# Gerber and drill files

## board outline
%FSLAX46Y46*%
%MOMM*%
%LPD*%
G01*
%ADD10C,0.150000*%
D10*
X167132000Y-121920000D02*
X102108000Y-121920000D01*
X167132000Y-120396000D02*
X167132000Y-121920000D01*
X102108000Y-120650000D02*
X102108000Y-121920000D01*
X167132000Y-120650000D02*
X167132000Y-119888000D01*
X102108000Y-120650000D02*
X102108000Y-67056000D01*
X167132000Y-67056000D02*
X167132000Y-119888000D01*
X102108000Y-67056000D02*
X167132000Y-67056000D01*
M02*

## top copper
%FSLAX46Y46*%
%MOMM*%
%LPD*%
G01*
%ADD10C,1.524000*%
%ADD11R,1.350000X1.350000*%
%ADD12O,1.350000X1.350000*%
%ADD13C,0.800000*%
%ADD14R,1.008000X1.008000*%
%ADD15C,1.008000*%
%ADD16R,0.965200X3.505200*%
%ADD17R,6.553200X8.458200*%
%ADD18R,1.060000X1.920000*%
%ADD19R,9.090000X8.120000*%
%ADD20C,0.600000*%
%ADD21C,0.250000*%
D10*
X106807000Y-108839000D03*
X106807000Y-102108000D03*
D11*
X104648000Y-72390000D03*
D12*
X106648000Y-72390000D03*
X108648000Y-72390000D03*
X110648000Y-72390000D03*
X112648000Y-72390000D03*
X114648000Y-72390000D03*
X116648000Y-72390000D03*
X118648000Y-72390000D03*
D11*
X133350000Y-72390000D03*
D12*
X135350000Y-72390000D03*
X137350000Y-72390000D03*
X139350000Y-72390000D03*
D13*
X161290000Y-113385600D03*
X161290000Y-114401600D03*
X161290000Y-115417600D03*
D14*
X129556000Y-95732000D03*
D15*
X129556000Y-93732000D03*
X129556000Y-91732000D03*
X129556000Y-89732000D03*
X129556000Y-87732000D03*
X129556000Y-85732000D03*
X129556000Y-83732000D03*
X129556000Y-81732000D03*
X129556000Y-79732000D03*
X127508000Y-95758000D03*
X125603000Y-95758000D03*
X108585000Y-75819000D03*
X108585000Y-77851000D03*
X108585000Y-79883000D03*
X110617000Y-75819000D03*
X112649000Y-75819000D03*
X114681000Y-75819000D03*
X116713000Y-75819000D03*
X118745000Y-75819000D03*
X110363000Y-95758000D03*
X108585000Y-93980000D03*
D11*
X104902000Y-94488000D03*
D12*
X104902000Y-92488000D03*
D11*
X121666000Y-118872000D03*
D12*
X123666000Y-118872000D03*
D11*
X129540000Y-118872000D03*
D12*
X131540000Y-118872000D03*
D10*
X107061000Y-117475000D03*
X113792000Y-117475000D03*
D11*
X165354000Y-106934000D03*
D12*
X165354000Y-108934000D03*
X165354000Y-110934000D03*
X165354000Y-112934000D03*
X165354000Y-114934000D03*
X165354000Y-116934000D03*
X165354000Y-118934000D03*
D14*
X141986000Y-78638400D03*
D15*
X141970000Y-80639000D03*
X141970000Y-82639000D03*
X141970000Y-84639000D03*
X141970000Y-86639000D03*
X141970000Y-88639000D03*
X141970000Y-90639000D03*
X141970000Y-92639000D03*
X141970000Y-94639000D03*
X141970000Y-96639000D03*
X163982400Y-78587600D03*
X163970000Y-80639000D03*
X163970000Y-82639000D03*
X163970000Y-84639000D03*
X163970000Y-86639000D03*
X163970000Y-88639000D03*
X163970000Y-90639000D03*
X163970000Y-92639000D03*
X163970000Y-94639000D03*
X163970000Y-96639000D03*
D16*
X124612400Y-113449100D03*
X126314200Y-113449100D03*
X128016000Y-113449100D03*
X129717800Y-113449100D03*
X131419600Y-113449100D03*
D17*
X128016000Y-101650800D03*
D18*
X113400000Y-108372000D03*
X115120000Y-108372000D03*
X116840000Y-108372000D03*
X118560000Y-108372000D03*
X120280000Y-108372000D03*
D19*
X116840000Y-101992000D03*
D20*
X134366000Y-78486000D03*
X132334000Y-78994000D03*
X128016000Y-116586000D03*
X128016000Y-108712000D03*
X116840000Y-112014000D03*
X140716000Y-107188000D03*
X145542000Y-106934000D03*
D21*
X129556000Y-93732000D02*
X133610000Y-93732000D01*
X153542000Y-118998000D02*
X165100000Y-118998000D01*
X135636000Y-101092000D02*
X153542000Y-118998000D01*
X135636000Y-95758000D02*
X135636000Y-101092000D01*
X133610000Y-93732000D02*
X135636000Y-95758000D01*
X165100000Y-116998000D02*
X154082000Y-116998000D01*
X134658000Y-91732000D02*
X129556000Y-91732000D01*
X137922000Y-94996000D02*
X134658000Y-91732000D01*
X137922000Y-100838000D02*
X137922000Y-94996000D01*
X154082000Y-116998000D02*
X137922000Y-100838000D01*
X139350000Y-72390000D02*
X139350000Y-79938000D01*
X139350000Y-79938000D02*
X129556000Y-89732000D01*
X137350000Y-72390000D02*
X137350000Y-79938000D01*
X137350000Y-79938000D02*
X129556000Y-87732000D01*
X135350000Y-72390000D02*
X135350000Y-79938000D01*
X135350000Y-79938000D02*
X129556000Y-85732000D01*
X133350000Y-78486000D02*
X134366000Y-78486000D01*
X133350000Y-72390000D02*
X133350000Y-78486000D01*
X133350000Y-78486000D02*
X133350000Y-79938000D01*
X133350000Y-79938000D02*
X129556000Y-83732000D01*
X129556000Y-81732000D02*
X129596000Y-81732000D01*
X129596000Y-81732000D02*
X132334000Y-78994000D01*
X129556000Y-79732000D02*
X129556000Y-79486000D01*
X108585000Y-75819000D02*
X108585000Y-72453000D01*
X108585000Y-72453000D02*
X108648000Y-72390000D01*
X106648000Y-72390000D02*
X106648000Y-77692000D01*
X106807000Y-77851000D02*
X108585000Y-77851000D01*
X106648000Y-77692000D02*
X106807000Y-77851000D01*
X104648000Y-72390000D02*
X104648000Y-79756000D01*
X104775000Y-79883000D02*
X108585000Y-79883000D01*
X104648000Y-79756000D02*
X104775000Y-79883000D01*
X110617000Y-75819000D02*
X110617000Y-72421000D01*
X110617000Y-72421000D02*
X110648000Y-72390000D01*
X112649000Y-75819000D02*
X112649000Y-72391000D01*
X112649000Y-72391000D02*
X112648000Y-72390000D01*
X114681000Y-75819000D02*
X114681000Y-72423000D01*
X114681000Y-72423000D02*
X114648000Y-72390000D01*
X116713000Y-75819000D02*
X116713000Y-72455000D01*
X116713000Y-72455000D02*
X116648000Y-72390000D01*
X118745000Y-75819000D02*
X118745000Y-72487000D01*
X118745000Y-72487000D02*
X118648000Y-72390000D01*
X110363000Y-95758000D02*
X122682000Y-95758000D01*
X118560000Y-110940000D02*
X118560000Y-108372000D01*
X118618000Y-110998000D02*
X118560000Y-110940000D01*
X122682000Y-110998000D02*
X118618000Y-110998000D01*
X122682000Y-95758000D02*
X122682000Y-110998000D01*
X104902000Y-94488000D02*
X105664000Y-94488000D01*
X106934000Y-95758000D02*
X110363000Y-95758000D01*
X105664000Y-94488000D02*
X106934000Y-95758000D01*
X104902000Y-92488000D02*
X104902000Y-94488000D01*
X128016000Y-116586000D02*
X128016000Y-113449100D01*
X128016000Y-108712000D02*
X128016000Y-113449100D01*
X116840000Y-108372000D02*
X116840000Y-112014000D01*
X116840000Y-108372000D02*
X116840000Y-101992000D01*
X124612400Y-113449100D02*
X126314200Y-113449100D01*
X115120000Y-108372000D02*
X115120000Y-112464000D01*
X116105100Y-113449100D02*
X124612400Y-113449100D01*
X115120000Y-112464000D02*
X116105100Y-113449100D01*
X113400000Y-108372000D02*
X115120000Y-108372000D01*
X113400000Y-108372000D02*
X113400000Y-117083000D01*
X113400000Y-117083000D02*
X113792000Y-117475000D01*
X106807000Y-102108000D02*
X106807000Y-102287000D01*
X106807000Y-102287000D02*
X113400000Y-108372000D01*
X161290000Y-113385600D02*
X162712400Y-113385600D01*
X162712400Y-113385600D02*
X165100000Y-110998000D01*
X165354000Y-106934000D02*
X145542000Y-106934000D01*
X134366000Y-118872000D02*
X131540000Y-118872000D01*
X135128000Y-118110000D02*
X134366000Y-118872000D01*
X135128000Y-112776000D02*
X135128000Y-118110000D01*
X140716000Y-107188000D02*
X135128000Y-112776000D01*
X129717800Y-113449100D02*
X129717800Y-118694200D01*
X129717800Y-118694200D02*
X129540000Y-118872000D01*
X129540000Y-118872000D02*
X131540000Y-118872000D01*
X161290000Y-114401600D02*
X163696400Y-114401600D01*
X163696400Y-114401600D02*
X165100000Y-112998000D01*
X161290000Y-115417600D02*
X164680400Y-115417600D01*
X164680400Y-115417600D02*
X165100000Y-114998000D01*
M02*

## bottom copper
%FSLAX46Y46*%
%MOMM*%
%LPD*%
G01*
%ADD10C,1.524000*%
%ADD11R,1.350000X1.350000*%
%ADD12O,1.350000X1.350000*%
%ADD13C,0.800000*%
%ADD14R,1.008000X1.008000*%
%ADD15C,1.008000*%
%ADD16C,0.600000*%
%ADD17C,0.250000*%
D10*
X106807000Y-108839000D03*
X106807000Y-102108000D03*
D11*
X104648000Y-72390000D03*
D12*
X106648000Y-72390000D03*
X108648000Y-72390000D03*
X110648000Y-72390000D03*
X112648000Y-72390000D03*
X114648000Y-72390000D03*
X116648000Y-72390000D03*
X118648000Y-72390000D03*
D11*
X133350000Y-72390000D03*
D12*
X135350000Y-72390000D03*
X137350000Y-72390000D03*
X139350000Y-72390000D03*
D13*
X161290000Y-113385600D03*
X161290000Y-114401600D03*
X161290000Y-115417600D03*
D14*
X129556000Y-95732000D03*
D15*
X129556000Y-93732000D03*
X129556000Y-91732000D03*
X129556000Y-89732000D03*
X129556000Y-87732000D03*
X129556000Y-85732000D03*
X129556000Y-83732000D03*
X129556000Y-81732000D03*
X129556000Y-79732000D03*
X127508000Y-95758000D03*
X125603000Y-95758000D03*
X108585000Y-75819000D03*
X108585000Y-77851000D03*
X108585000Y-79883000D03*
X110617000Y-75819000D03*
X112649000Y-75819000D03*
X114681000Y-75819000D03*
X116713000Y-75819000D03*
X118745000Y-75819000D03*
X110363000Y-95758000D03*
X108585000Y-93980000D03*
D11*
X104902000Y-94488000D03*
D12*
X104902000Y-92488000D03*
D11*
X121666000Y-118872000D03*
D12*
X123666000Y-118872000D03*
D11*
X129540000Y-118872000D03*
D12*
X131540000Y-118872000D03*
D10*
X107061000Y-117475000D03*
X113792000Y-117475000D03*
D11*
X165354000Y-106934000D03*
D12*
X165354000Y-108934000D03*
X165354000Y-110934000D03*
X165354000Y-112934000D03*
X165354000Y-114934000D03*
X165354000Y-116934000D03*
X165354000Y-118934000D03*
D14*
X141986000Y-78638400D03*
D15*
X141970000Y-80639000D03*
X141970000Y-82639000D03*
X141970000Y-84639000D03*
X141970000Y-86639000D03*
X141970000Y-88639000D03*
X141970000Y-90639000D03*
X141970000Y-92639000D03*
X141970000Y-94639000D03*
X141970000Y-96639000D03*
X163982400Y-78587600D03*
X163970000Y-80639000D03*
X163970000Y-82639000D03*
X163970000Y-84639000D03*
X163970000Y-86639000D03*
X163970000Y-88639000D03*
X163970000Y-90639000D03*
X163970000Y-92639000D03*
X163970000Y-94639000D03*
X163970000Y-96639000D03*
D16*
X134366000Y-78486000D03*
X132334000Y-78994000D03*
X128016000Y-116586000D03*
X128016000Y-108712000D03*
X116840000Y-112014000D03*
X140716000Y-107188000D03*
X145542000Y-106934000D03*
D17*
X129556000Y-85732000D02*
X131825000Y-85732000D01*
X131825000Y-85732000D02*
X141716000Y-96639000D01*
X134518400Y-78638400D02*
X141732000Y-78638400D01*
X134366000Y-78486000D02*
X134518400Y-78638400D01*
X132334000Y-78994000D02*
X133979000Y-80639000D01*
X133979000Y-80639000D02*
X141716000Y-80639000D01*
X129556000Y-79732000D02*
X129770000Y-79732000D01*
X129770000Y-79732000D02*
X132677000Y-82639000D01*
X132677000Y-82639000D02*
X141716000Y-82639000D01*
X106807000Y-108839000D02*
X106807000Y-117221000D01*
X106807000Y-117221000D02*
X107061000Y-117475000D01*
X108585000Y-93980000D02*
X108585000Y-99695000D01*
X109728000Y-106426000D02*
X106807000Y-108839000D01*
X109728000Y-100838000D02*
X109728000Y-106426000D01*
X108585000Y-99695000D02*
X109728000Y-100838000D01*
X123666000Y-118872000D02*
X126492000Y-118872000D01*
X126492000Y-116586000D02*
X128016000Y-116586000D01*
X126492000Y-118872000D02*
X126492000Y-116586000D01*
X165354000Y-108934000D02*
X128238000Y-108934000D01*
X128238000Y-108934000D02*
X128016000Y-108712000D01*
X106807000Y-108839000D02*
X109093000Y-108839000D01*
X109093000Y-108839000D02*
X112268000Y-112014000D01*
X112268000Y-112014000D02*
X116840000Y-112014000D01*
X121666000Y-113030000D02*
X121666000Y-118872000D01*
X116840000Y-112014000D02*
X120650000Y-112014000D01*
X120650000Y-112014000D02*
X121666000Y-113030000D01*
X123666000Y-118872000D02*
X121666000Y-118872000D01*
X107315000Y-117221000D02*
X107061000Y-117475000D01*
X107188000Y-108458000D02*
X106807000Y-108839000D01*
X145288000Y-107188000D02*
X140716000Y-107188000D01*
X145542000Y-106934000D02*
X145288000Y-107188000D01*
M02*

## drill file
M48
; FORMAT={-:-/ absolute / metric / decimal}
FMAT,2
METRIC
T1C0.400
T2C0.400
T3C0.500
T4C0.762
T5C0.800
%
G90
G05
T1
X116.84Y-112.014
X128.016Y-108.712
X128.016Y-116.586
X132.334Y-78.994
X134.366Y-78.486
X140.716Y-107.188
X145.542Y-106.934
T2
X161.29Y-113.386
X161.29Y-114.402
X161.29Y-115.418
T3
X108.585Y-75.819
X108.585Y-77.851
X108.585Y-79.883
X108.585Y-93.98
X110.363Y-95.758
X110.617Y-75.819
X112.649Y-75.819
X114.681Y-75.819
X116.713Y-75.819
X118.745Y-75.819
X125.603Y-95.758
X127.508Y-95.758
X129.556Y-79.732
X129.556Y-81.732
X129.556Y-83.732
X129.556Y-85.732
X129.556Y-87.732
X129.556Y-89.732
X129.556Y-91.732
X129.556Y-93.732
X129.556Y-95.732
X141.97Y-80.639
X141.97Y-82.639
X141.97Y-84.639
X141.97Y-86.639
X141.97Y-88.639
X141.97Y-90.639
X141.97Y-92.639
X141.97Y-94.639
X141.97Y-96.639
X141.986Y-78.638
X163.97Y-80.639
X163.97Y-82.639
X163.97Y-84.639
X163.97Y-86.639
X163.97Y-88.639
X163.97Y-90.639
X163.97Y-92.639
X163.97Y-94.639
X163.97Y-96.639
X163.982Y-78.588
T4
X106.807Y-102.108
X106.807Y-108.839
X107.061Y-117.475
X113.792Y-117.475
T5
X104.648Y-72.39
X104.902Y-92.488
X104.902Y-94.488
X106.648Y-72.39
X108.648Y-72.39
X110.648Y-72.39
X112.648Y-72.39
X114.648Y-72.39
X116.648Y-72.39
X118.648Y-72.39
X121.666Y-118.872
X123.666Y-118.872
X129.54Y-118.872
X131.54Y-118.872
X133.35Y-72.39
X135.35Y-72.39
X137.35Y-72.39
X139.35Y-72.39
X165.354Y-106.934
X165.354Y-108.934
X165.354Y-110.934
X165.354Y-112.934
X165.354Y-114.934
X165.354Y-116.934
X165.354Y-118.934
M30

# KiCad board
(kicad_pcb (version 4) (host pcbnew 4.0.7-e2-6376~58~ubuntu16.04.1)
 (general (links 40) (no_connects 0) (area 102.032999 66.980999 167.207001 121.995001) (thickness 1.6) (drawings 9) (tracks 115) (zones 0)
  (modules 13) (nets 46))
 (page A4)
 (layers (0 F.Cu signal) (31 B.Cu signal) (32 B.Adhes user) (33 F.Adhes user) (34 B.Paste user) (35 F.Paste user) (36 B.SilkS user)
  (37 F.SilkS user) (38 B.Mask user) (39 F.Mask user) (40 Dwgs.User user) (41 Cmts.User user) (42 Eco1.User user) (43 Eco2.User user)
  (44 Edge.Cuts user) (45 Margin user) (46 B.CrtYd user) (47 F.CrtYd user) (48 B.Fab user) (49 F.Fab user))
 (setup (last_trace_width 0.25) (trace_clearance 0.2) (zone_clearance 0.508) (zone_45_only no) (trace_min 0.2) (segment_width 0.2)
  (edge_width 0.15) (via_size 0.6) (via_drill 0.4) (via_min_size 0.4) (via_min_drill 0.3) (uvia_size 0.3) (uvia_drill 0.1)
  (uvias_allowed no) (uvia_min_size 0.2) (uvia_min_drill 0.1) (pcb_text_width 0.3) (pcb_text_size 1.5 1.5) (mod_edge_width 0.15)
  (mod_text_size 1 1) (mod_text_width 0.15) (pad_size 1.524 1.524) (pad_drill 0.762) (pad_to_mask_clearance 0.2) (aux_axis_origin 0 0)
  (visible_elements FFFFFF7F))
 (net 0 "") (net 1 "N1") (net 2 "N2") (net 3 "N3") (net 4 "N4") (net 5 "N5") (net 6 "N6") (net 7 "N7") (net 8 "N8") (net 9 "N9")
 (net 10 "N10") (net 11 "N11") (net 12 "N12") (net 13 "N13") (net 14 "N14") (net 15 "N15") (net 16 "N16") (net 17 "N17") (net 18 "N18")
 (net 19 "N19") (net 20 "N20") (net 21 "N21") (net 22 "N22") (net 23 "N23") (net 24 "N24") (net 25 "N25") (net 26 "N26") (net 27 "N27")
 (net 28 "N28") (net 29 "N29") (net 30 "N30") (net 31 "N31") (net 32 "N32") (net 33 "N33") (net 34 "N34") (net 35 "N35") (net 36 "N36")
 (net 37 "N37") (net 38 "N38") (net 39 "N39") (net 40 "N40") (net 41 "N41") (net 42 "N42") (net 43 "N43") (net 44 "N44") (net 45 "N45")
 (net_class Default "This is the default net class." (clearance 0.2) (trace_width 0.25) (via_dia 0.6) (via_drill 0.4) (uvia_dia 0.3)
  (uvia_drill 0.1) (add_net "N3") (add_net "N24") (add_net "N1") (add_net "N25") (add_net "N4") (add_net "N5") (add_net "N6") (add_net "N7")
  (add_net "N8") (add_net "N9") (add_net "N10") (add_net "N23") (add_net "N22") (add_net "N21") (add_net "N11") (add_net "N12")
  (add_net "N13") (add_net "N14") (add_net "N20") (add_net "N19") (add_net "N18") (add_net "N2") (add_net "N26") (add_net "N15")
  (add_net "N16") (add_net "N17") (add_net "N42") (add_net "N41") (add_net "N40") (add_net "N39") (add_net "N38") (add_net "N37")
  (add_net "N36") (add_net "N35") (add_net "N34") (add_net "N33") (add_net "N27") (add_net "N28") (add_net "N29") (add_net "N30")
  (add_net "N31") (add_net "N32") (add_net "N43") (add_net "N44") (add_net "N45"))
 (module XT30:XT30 (layer F.Cu) (at 100.838 107.442 90)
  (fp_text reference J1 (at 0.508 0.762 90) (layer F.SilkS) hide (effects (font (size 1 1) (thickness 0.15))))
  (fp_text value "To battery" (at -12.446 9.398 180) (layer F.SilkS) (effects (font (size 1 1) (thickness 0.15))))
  (pad 1 thru_hole circle (at -1.397 5.969 90) (size 1.524 1.524) (drill 0.762) (layers *.Cu *.Mask) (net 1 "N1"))
  (pad 2 thru_hole circle (at 5.334 5.969 90) (size 1.524 1.524) (drill 0.762) (layers *.Cu *.Mask) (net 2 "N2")))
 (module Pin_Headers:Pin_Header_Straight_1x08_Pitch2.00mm (layer F.Cu) (at 104.648 72.39 90)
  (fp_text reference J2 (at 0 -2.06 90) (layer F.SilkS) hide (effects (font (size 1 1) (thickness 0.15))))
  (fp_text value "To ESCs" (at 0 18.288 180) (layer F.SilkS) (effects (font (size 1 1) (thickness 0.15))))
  (pad 1 thru_hole rect (at 0 0 90) (size 1.35 1.35) (drill 0.8) (layers *.Cu *.Mask) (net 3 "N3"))
  (pad 2 thru_hole oval (at 0 2 90) (size 1.35 1.35) (drill 0.8) (layers *.Cu *.Mask) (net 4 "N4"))
  (pad 3 thru_hole oval (at 0 4 90) (size 1.35 1.35) (drill 0.8) (layers *.Cu *.Mask) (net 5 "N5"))
  (pad 4 thru_hole oval (at 0 6 90) (size 1.35 1.35) (drill 0.8) (layers *.Cu *.Mask) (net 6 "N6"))
  (pad 5 thru_hole oval (at 0 8 90) (size 1.35 1.35) (drill 0.8) (layers *.Cu *.Mask) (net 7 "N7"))
  (pad 6 thru_hole oval (at 0 10 90) (size 1.35 1.35) (drill 0.8) (layers *.Cu *.Mask) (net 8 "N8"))
  (pad 7 thru_hole oval (at 0 12 90) (size 1.35 1.35) (drill 0.8) (layers *.Cu *.Mask) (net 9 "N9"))
  (pad 8 thru_hole oval (at 0 14 90) (size 1.35 1.35) (drill 0.8) (layers *.Cu *.Mask) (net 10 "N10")))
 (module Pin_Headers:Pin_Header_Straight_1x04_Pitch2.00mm (layer F.Cu) (at 133.35 72.39 90)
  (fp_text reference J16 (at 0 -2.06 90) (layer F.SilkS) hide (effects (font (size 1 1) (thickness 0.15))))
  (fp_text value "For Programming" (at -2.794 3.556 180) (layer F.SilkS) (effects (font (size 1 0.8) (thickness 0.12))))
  (pad 1 thru_hole rect (at 0 0 90) (size 1.35 1.35) (drill 0.8) (layers *.Cu *.Mask) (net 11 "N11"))
  (pad 2 thru_hole oval (at 0 2 90) (size 1.35 1.35) (drill 0.8) (layers *.Cu *.Mask) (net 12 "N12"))
  (pad 3 thru_hole oval (at 0 4 90) (size 1.35 1.35) (drill 0.8) (layers *.Cu *.Mask) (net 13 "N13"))
  (pad 4 thru_hole oval (at 0 6 90) (size 1.35 1.35) (drill 0.8) (layers *.Cu *.Mask) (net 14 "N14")))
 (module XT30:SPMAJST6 (layer F.Cu) (at 164.084 115.316 270)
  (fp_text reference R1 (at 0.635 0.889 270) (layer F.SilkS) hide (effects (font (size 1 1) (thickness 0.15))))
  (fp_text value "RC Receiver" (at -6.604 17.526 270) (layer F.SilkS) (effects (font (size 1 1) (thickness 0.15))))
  (pad 1 thru_hole circle (at -1.9304 2.794 270) (size 0.8 0.8) (drill 0.4) (layers *.Cu *.Mask) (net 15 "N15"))
  (pad 2 thru_hole circle (at -0.9144 2.794 270) (size 0.8 0.8) (drill 0.4) (layers *.Cu *.Mask) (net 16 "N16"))
  (pad 3 thru_hole circle (at 0.1016 2.794 270) (size 0.8 0.8) (drill 0.4) (layers *.Cu *.Mask) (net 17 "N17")))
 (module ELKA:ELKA (layer F.Cu) (at 118.11 72.39 180)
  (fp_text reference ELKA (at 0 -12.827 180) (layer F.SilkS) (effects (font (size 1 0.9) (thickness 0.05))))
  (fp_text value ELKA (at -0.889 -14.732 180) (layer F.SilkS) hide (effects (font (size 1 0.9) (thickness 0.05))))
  (pad I thru_hole rect (at -11.446 -23.342 180) (size 1.008 1.008) (drill 0.5) (layers *.Cu *.Mask F.SilkS) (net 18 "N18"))
  (pad H thru_hole circle (at -11.446 -21.342 180) (size 1.008 1.008) (drill 0.5) (layers *.Cu *.Mask F.SilkS) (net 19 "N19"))
  (pad G thru_hole circle (at -11.446 -19.342 180) (size 1.008 1.008) (drill 0.5) (layers *.Cu *.Mask F.SilkS) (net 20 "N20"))
  (pad F thru_hole circle (at -11.446 -17.342 180) (size 1.008 1.008) (drill 0.5) (layers *.Cu *.Mask F.SilkS) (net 14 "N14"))
  (pad E thru_hole circle (at -11.446 -15.342 180) (size 1.008 1.008) (drill 0.5) (layers *.Cu *.Mask F.SilkS) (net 13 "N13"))
  (pad D thru_hole circle (at -11.446 -13.342 180) (size 1.008 1.008) (drill 0.5) (layers *.Cu *.Mask F.SilkS) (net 12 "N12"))
  (pad C thru_hole circle (at -11.446 -11.342 180) (size 1.008 1.008) (drill 0.5) (layers *.Cu *.Mask F.SilkS) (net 11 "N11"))
  (pad B thru_hole circle (at -11.446 -9.342 180) (size 1.008 1.008) (drill 0.5) (layers *.Cu *.Mask F.SilkS) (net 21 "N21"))
  (pad A thru_hole circle (at -11.446 -7.342 180) (size 1.008 1.008) (drill 0.5) (layers *.Cu *.Mask F.SilkS) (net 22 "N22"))
  (pad 9 thru_hole circle (at -9.398 -23.368 180) (size 1.008 1.008) (drill 0.5) (layers *.Cu *.Mask F.SilkS) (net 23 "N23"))
  (pad 10 thru_hole circle (at -7.493 -23.368 180) (size 1.008 1.008) (drill 0.5) (layers *.Cu *.Mask F.SilkS) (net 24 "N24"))
  (pad 3 thru_hole circle (at 9.525 -3.429 180) (size 1.008 1.008) (drill 0.5) (layers *.Cu *.Mask F.SilkS) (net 5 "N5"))
  (pad 2 thru_hole circle (at 9.525 -5.461 180) (size 1.008 1.008) (drill 0.5) (layers *.Cu *.Mask F.SilkS) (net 4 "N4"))
  (pad 1 thru_hole circle (at 9.525 -7.493 180) (size 1.008 1.008) (drill 0.5) (layers *.Cu *.Mask F.SilkS) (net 3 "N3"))
  (pad 4 thru_hole circle (at 7.493 -3.429 180) (size 1.008 1.008) (drill 0.5) (layers *.Cu *.Mask F.SilkS) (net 6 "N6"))
  (pad 5 thru_hole circle (at 5.461 -3.429 180) (size 1.008 1.008) (drill 0.5) (layers *.Cu *.Mask F.SilkS) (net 7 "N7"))
  (pad 6 thru_hole circle (at 3.429 -3.429 180) (size 1.008 1.008) (drill 0.5) (layers *.Cu *.Mask F.SilkS) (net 8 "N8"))
  (pad 7 thru_hole circle (at 1.397 -3.429 180) (size 1.008 1.008) (drill 0.5) (layers *.Cu *.Mask F.SilkS) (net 9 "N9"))
  (pad 8 thru_hole circle (at -0.635 -3.429 180) (size 1.008 1.008) (drill 0.5) (layers *.Cu *.Mask F.SilkS) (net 10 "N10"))
  (pad 12 thru_hole circle (at 7.747 -23.368 180) (size 1.008 1.008) (drill 0.5) (layers *.Cu *.Mask F.SilkS) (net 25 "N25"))
  (pad 11 thru_hole circle (at 9.525 -21.59 180) (size 1.008 1.008) (drill 0.5) (layers *.Cu *.Mask F.SilkS) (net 1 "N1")))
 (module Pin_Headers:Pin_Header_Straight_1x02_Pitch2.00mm (layer F.Cu) (at 104.902 94.488 180)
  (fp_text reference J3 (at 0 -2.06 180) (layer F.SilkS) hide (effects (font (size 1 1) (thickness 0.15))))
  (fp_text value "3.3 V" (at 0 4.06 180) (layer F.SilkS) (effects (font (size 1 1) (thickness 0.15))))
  (pad 1 thru_hole rect (at 0 0 180) (size 1.35 1.35) (drill 0.8) (layers *.Cu *.Mask) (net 25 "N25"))
  (pad 2 thru_hole oval (at 0 2 180) (size 1.35 1.35) (drill 0.8) (layers *.Cu *.Mask) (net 25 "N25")))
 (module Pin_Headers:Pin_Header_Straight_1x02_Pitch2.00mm (layer F.Cu) (at 121.666 118.872 90)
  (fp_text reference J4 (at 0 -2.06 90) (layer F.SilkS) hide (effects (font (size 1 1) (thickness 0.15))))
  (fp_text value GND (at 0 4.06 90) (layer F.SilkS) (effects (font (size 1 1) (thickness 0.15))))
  (pad 1 thru_hole rect (at 0 0 90) (size 1.35 1.35) (drill 0.8) (layers *.Cu *.Mask) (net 1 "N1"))
  (pad 2 thru_hole oval (at 0 2 90) (size 1.35 1.35) (drill 0.8) (layers *.Cu *.Mask) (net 1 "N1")))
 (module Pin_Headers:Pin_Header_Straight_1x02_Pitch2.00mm (layer F.Cu) (at 129.54 118.872 90)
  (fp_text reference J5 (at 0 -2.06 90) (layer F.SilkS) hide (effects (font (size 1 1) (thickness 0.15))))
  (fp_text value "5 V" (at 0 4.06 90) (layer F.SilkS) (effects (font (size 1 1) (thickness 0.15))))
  (pad 1 thru_hole rect (at 0 0 90) (size 1.35 1.35) (drill 0.8) (layers *.Cu *.Mask) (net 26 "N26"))
  (pad 2 thru_hole oval (at 0 2 90) (size 1.35 1.35) (drill 0.8) (layers *.Cu *.Mask) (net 26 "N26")))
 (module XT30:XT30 (layer F.Cu) (at 108.458 111.506)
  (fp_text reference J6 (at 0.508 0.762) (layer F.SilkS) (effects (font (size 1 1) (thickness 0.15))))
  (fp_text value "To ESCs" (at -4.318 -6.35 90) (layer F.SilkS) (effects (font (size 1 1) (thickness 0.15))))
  (pad 1 thru_hole circle (at -1.397 5.969) (size 1.524 1.524) (drill 0.762) (layers *.Cu *.Mask) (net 1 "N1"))
  (pad 2 thru_hole circle (at 5.334 5.969) (size 1.524 1.524) (drill 0.762) (layers *.Cu *.Mask) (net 2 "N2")))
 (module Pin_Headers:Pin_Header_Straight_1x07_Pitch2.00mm (layer F.Cu) (at 165.354 106.934)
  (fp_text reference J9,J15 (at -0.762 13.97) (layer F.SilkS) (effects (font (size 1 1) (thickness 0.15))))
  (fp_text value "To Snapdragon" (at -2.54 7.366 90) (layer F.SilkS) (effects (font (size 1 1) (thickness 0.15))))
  (pad 1 thru_hole rect (at 0 0) (size 1.35 1.35) (drill 0.8) (layers *.Cu *.Mask) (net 26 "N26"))
  (pad 2 thru_hole oval (at 0 2) (size 1.35 1.35) (drill 0.8) (layers *.Cu *.Mask) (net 1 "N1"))
  (pad 3 thru_hole oval (at 0 4) (size 1.35 1.35) (drill 0.8) (layers *.Cu *.Mask) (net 15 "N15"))
  (pad 4 thru_hole oval (at 0 6) (size 1.35 1.35) (drill 0.8) (layers *.Cu *.Mask) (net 16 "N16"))
  (pad 5 thru_hole oval (at 0 8) (size 1.35 1.35) (drill 0.8) (layers *.Cu *.Mask) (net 17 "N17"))
  (pad 6 thru_hole oval (at 0 10) (size 1.35 1.35) (drill 0.8) (layers *.Cu *.Mask) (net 20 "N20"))
  (pad 7 thru_hole oval (at 0 12) (size 1.35 1.35) (drill 0.8) (layers *.Cu *.Mask) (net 19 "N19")))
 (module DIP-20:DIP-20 (layer F.Cu) (at 140.716 104.648)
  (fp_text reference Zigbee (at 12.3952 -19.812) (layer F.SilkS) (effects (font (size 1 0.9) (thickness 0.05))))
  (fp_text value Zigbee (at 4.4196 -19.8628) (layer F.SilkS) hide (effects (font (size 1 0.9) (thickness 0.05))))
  (pad 1 thru_hole rect (at 1.27 -26.0096) (size 1.008 1.008) (drill 0.5) (layers *.Cu *.Mask F.SilkS) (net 11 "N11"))
  (pad 2 thru_hole circle (at 1.254 -24.009) (size 1.008 1.008) (drill 0.5) (layers *.Cu *.Mask F.SilkS) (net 21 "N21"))
  (pad 3 thru_hole circle (at 1.254 -22.009) (size 1.008 1.008) (drill 0.5) (layers *.Cu *.Mask F.SilkS) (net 22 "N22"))
  (pad 4 thru_hole circle (at 1.254 -20.009) (size 1.008 1.008) (drill 0.5) (layers *.Cu *.Mask F.SilkS) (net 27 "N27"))
  (pad 5 thru_hole circle (at 1.254 -18.009) (size 1.008 1.008) (drill 0.5) (layers *.Cu *.Mask F.SilkS) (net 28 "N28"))
  (pad 6 thru_hole circle (at 1.254 -16.009) (size 1.008 1.008) (drill 0.5) (layers *.Cu *.Mask F.SilkS) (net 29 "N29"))
  (pad 7 thru_hole circle (at 1.254 -14.009) (size 1.008 1.008) (drill 0.5) (layers *.Cu *.Mask F.SilkS) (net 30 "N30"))
  (pad 8 thru_hole circle (at 1.254 -12.009) (size 1.008 1.008) (drill 0.5) (layers *.Cu *.Mask F.SilkS) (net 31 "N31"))
  (pad 9 thru_hole circle (at 1.254 -10.009) (size 1.008 1.008) (drill 0.5) (layers *.Cu *.Mask F.SilkS) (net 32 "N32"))
  (pad 10 thru_hole circle (at 1.254 -8.009) (size 1.008 1.008) (drill 0.5) (layers *.Cu *.Mask F.SilkS) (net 12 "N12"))
  (pad 20 thru_hole circle (at 23.2664 -26.0604) (size 1.008 1.008) (drill 0.5) (layers *.Cu *.Mask F.SilkS) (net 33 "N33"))
  (pad 19 thru_hole circle (at 23.254 -24.009) (size 1.008 1.008) (drill 0.5) (layers *.Cu *.Mask F.SilkS) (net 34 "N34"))
  (pad 18 thru_hole circle (at 23.254 -22.009) (size 1.008 1.008) (drill 0.5) (layers *.Cu *.Mask F.SilkS) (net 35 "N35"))
  (pad 17 thru_hole circle (at 23.254 -20.009) (size 1.008 1.008) (drill 0.5) (layers *.Cu *.Mask F.SilkS) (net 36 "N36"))
  (pad 16 thru_hole circle (at 23.254 -18.009) (size 1.008 1.008) (drill 0.5) (layers *.Cu *.Mask F.SilkS) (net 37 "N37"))
  (pad 15 thru_hole circle (at 23.254 -16.009) (size 1.008 1.008) (drill 0.5) (layers *.Cu *.Mask F.SilkS) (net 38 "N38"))
  (pad 14 thru_hole circle (at 23.254 -14.009) (size 1.008 1.008) (drill 0.5) (layers *.Cu *.Mask F.SilkS) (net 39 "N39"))
  (pad 13 thru_hole circle (at 23.254 -12.009) (size 1.008 1.008) (drill 0.5) (layers *.Cu *.Mask F.SilkS) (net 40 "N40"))
  (pad 12 thru_hole circle (at 23.254 -10.009) (size 1.008 1.008) (drill 0.5) (layers *.Cu *.Mask F.SilkS) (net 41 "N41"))
  (pad 11 thru_hole circle (at 23.254 -8.009) (size 1.008 1.008) (drill 0.5) (layers *.Cu *.Mask F.SilkS) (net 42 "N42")))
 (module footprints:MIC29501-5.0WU (layer F.Cu) (at 128.016 104.394)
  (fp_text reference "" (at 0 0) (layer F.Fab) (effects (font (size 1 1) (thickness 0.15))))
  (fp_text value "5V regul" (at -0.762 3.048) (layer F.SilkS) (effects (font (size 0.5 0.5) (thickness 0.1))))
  (pad 1 smd rect (at -3.4036 9.0551) (size 0.9652 3.5052) (layers F.Cu F.Paste F.Mask) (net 2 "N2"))
  (pad 2 smd rect (at -1.7018 9.0551) (size 0.9652 3.5052) (layers F.Cu F.Paste F.Mask) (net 2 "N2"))
  (pad 3 smd rect (at 0 9.0551) (size 0.9652 3.5052) (layers F.Cu F.Paste F.Mask) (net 1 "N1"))
  (pad 4 smd rect (at 1.7018 9.0551) (size 0.9652 3.5052) (layers F.Cu F.Paste F.Mask) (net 26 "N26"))
  (pad 5 smd rect (at 3.4036 9.0551) (size 0.9652 3.5052) (layers F.Cu F.Paste F.Mask) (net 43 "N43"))
  (pad 6 smd rect (at 0 -2.7432) (size 6.5532 8.4582) (layers F.Cu F.Paste F.Mask) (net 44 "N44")))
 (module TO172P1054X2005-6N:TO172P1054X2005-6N (layer F.Cu) (at 116.84 103.632)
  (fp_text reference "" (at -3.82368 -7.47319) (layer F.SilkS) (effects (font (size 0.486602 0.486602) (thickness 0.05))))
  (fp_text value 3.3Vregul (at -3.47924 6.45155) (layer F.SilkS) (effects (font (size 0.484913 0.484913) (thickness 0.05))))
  (pad 1 smd rect (at -3.44 4.74 90) (size 1.92 1.06) (layers F.Cu F.Paste F.Mask) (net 2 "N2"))
  (pad 2 smd rect (at -1.72 4.74 90) (size 1.92 1.06) (layers F.Cu F.Paste F.Mask) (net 2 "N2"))
  (pad 3 smd rect (at 0 4.74 90) (size 1.92 1.06) (layers F.Cu F.Paste F.Mask) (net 1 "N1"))
  (pad 4 smd rect (at 1.72 4.74 90) (size 1.92 1.06) (layers F.Cu F.Paste F.Mask) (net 25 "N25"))
  (pad 5 smd rect (at 3.44 4.74 90) (size 1.92 1.06) (layers F.Cu F.Paste F.Mask) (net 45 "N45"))
  (pad 6 smd rect (at 0 -1.64 90) (size 8.12 9.09) (layers F.Cu F.Paste F.Mask) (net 1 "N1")))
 (gr_line (start 167.132 121.92) (end 102.108 121.92) (angle 90) (layer Edge.Cuts) (width 0.15))
 (gr_line (start 167.132 120.396) (end 167.132 121.92) (angle 90) (layer Edge.Cuts) (width 0.15))
 (gr_line (start 102.108 120.65) (end 102.108 121.92) (angle 90) (layer Edge.Cuts) (width 0.15))
 (gr_line (start 167.132 120.65) (end 167.132 119.888) (angle 90) (layer Edge.Cuts) (width 0.15))
 (gr_line (start 102.108 120.65) (end 102.108 67.056) (angle 90) (layer Edge.Cuts) (width 0.15))
 (gr_line (start 167.132 67.056) (end 167.132 119.888) (angle 90) (layer Edge.Cuts) (width 0.15))
 (gr_line (start 102.108 67.056) (end 167.132 67.056) (angle 90) (layer Edge.Cuts) (width 0.15))
 (segment (start 129.556 93.732) (end 133.61 93.732) (width 0.25) (layer F.Cu) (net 19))
 (segment (start 153.542 118.998) (end 165.1 118.998) (width 0.25) (layer F.Cu) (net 19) (status 20))
 (segment (start 135.636 101.092) (end 153.542 118.998) (width 0.25) (layer F.Cu) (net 19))
 (segment (start 135.636 95.758) (end 135.636 101.092) (width 0.25) (layer F.Cu) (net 19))
 (segment (start 133.61 93.732) (end 135.636 95.758) (width 0.25) (layer F.Cu) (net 19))
 (segment (start 165.1 116.998) (end 154.082 116.998) (width 0.25) (layer F.Cu) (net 20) (status 10))
 (segment (start 134.658 91.732) (end 129.556 91.732) (width 0.25) (layer F.Cu) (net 20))
 (segment (start 137.922 94.996) (end 134.658 91.732) (width 0.25) (layer F.Cu) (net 20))
 (segment (start 137.922 100.838) (end 137.922 94.996) (width 0.25) (layer F.Cu) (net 20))
 (segment (start 154.082 116.998) (end 137.922 100.838) (width 0.25) (layer F.Cu) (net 20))
 (segment (start 139.35 72.39) (end 139.35 79.938) (width 0.25) (layer F.Cu) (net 14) (status 10))
 (segment (start 139.35 79.938) (end 129.556 89.732) (width 0.25) (layer F.Cu) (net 14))
 (segment (start 137.35 72.39) (end 137.35 79.938) (width 0.25) (layer F.Cu) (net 13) (status 10))
 (segment (start 137.35 79.938) (end 129.556 87.732) (width 0.25) (layer F.Cu) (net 13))
 (segment (start 129.556 85.732) (end 131.825 85.732) (width 0.25) (layer B.Cu) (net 12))
 (segment (start 131.825 85.732) (end 141.716 96.639) (width 0.25) (layer B.Cu) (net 12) (status 20))
 (segment (start 135.35 72.39) (end 135.35 79.938) (width 0.25) (layer F.Cu) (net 12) (status 10))
 (segment (start 135.35 79.938) (end 129.556 85.732) (width 0.25) (layer F.Cu) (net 12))
 (segment (start 133.35 78.486) (end 134.366 78.486) (width 0.25) (layer F.Cu) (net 11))
 (segment (start 134.5184 78.6384) (end 141.732 78.6384) (width 0.25) (layer B.Cu) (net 11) (status 20))
 (segment (start 134.366 78.486) (end 134.5184 78.6384) (width 0.25) (layer B.Cu) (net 11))
 (via (at 134.366 78.486) (size 0.6) (drill 0.4) (layers F.Cu B.Cu) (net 11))
 (segment (start 133.35 72.39) (end 133.35 78.486) (width 0.25) (layer F.Cu) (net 11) (status 10))
 (segment (start 133.35 78.486) (end 133.35 79.938) (width 0.25) (layer F.Cu) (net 11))
 (segment (start 133.35 79.938) (end 129.556 83.732) (width 0.25) (layer F.Cu) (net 11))
 (segment (start 129.556 81.732) (end 129.596 81.732) (width 0.25) (layer F.Cu) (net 21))
 (segment (start 129.596 81.732) (end 132.334 78.994) (width 0.25) (layer F.Cu) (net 21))
 (via (at 132.334 78.994) (size 0.6) (drill 0.4) (layers F.Cu B.Cu) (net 21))
 (segment (start 132.334 78.994) (end 133.979 80.639) (width 0.25) (layer B.Cu) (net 21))
 (segment (start 133.979 80.639) (end 141.716 80.639) (width 0.25) (layer B.Cu) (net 21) (status 20))
 (segment (start 129.556 79.732) (end 129.77 79.732) (width 0.25) (layer B.Cu) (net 22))
 (segment (start 129.77 79.732) (end 132.677 82.639) (width 0.25) (layer B.Cu) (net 22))
 (segment (start 132.677 82.639) (end 141.716 82.639) (width 0.25) (layer B.Cu) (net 22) (status 20))
 (segment (start 129.556 79.732) (end 129.556 79.486) (width 0.25) (layer F.Cu) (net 22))
 (segment (start 108.585 75.819) (end 108.585 72.453) (width 0.25) (layer F.Cu) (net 5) (status 20))
 (segment (start 108.585 72.453) (end 108.648 72.39) (width 0.25) (layer F.Cu) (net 5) (status 30))
 (segment (start 106.648 72.39) (end 106.648 77.692) (width 0.25) (layer F.Cu) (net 4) (status 10))
 (segment (start 106.807 77.851) (end 108.585 77.851) (width 0.25) (layer F.Cu) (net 4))
 (segment (start 106.648 77.692) (end 106.807 77.851) (width 0.25) (layer F.Cu) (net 4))
 (segment (start 104.648 72.39) (end 104.648 79.756) (width 0.25) (layer F.Cu) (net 3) (status 10))
 (segment (start 104.775 79.883) (end 108.585 79.883) (width 0.25) (layer F.Cu) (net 3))
 (segment (start 104.648 79.756) (end 104.775 79.883) (width 0.25) (layer F.Cu) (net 3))
 (segment (start 110.617 75.819) (end 110.617 72.421) (width 0.25) (layer F.Cu) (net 6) (status 20))
 (segment (start 110.617 72.421) (end 110.648 72.39) (width 0.25) (layer F.Cu) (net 6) (status 30))
 (segment (start 112.649 75.819) (end 112.649 72.391) (width 0.25) (layer F.Cu) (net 7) (status 20))
 (segment (start 112.649 72.391) (end 112.648 72.39) (width 0.25) (layer F.Cu) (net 7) (status 30))
 (segment (start 114.681 75.819) (end 114.681 72.423) (width 0.25) (layer F.Cu) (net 8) (status 20))
 (segment (start 114.681 72.423) (end 114.648 72.39) (width 0.25) (layer F.Cu) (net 8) (status 30))
 (segment (start 116.713 75.819) (end 116.713 72.455) (width 0.25) (layer F.Cu) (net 9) (status 20))
 (segment (start 116.713 72.455) (end 116.648 72.39) (width 0.25) (layer F.Cu) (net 9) (status 30))
 (segment (start 118.745 75.819) (end 118.745 72.487) (width 0.25) (layer F.Cu) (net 10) (status 20))
 (segment (start 118.745 72.487) (end 118.648 72.39) (width 0.25) (layer F.Cu) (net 10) (status 30))
 (segment (start 110.363 95.758) (end 122.682 95.758) (width 0.25) (layer F.Cu) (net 25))
 (segment (start 118.56 110.94) (end 118.56 108.372) (width 0.25) (layer F.Cu) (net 25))
 (segment (start 118.618 110.998) (end 118.56 110.94) (width 0.25) (layer F.Cu) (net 25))
 (segment (start 122.682 110.998) (end 118.618 110.998) (width 0.25) (layer F.Cu) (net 25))
 (segment (start 122.682 95.758) (end 122.682 110.998) (width 0.25) (layer F.Cu) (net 25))
 (segment (start 104.902 94.488) (end 105.664 94.488) (width 0.25) (layer F.Cu) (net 25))
 (segment (start 106.934 95.758) (end 110.363 95.758) (width 0.25) (layer F.Cu) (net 25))
 (segment (start 105.664 94.488) (end 106.934 95.758) (width 0.25) (layer F.Cu) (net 25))
 (segment (start 104.902 92.488) (end 104.902 94.488) (width 0.25) (layer F.Cu) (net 25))
 (segment (start 106.807 108.839) (end 106.807 117.221) (width 0.25) (layer B.Cu) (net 1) (status C00000))
 (segment (start 106.807 117.221) (end 107.061 117.475) (width 0.25) (layer B.Cu) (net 1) (status C00000))
 (segment (start 108.585 93.98) (end 108.585 99.695) (width 0.25) (layer B.Cu) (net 1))
 (segment (start 109.728 106.426) (end 106.807 108.839) (width 0.25) (layer B.Cu) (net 1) (status 20))
 (segment (start 109.728 100.838) (end 109.728 106.426) (width 0.25) (layer B.Cu) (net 1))
 (segment (start 108.585 99.695) (end 109.728 100.838) (width 0.25) (layer B.Cu) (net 1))
 (segment (start 123.666 118.872) (end 126.492 118.872) (width 0.25) (layer B.Cu) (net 1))
 (segment (start 128.016 116.586) (end 128.016 113.4491) (width 0.25) (layer F.Cu) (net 1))
 (via (at 128.016 116.586) (size 0.6) (drill 0.4) (layers F.Cu B.Cu) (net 1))
 (segment (start 126.492 116.586) (end 128.016 116.586) (width 0.25) (layer B.Cu) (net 1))
 (segment (start 126.492 118.872) (end 126.492 116.586) (width 0.25) (layer B.Cu) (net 1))
 (segment (start 165.354 108.934) (end 128.238 108.934) (width 0.25) (layer B.Cu) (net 1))
 (segment (start 128.238 108.934) (end 128.016 108.712) (width 0.25) (layer B.Cu) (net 1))
 (via (at 128.016 108.712) (size 0.6) (drill 0.4) (layers F.Cu B.Cu) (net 1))
 (segment (start 128.016 108.712) (end 128.016 113.4491) (width 0.25) (layer F.Cu) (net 1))
 (segment (start 116.84 108.372) (end 116.84 112.014) (width 0.25) (layer F.Cu) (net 1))
 (via (at 116.84 112.014) (size 0.6) (drill 0.4) (layers F.Cu B.Cu) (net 1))
 (segment (start 106.807 108.839) (end 109.093 108.839) (width 0.25) (layer B.Cu) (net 1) (status 10))
 (segment (start 109.093 108.839) (end 112.268 112.014) (width 0.25) (layer B.Cu) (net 1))
 (segment (start 112.268 112.014) (end 116.84 112.014) (width 0.25) (layer B.Cu) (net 1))
 (segment (start 121.666 113.03) (end 121.666 118.872) (width 0.25) (layer B.Cu) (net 1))
 (segment (start 116.84 112.014) (end 120.65 112.014) (width 0.25) (layer B.Cu) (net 1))
 (segment (start 120.65 112.014) (end 121.666 113.03) (width 0.25) (layer B.Cu) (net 1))
 (segment (start 123.666 118.872) (end 121.666 118.872) (width 0.25) (layer B.Cu) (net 1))
 (segment (start 107.315 117.221) (end 107.061 117.475) (width 0.25) (layer B.Cu) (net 1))
 (segment (start 107.188 108.458) (end 106.807 108.839) (width 0.25) (layer B.Cu) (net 1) (status 30))
 (segment (start 116.84 108.372) (end 116.84 101.992) (width 0.25) (layer F.Cu) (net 1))
 (segment (start 124.6124 113.4491) (end 126.3142 113.4491) (width 0.25) (layer F.Cu) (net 2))
 (segment (start 115.12 108.372) (end 115.12 112.464) (width 0.25) (layer F.Cu) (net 2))
 (segment (start 116.1051 113.4491) (end 124.6124 113.4491) (width 0.25) (layer F.Cu) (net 2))
 (segment (start 115.12 112.464) (end 116.1051 113.4491) (width 0.25) (layer F.Cu) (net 2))
 (segment (start 113.4 108.372) (end 115.12 108.372) (width 0.25) (layer F.Cu) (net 2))
 (segment (start 113.4 108.372) (end 113.4 117.083) (width 0.25) (layer F.Cu) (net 2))
 (segment (start 113.4 117.083) (end 113.792 117.475) (width 0.25) (layer F.Cu) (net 2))
 (segment (start 106.807 102.108) (end 106.807 102.287) (width 0.25) (layer F.Cu) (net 2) (status 30))
 (segment (start 106.807 102.287) (end 113.4 108.372) (width 0.25) (layer F.Cu) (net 2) (status 10))
 (segment (start 161.29 113.3856) (end 162.7124 113.3856) (width 0.25) (layer F.Cu) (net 15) (status 10))
 (segment (start 162.7124 113.3856) (end 165.1 110.998) (width 0.25) (layer F.Cu) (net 15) (status 20))
 (segment (start 165.354 106.934) (end 145.542 106.934) (width 0.25) (layer F.Cu) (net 26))
 (segment (start 134.366 118.872) (end 131.54 118.872) (width 0.25) (layer F.Cu) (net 26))
 (segment (start 135.128 118.11) (end 134.366 118.872) (width 0.25) (layer F.Cu) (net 26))
 (segment (start 135.128 112.776) (end 135.128 118.11) (width 0.25) (layer F.Cu) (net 26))
 (segment (start 140.716 107.188) (end 135.128 112.776) (width 0.25) (layer F.Cu) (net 26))
 (via (at 140.716 107.188) (size 0.6) (drill 0.4) (layers F.Cu B.Cu) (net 26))
 (segment (start 145.288 107.188) (end 140.716 107.188) (width 0.25) (layer B.Cu) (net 26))
 (segment (start 145.542 106.934) (end 145.288 107.188) (width 0.25) (layer B.Cu) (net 26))
 (via (at 145.542 106.934) (size 0.6) (drill 0.4) (layers F.Cu B.Cu) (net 26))
 (segment (start 129.7178 113.4491) (end 129.7178 118.6942) (width 0.25) (layer F.Cu) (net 26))
 (segment (start 129.7178 118.6942) (end 129.54 118.872) (width 0.25) (layer F.Cu) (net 26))
 (segment (start 129.54 118.872) (end 131.54 118.872) (width 0.25) (layer F.Cu) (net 26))
 (segment (start 161.29 114.4016) (end 163.6964 114.4016) (width 0.25) (layer F.Cu) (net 16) (status 10))
 (segment (start 163.6964 114.4016) (end 165.1 112.998) (width 0.25) (layer F.Cu) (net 16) (status 20))
 (segment (start 161.29 115.4176) (end 164.6804 115.4176) (width 0.25) (layer F.Cu) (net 17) (status 10))
 (segment (start 164.6804 115.4176) (end 165.1 114.998) (width 0.25) (layer F.Cu) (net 17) (status 30)))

